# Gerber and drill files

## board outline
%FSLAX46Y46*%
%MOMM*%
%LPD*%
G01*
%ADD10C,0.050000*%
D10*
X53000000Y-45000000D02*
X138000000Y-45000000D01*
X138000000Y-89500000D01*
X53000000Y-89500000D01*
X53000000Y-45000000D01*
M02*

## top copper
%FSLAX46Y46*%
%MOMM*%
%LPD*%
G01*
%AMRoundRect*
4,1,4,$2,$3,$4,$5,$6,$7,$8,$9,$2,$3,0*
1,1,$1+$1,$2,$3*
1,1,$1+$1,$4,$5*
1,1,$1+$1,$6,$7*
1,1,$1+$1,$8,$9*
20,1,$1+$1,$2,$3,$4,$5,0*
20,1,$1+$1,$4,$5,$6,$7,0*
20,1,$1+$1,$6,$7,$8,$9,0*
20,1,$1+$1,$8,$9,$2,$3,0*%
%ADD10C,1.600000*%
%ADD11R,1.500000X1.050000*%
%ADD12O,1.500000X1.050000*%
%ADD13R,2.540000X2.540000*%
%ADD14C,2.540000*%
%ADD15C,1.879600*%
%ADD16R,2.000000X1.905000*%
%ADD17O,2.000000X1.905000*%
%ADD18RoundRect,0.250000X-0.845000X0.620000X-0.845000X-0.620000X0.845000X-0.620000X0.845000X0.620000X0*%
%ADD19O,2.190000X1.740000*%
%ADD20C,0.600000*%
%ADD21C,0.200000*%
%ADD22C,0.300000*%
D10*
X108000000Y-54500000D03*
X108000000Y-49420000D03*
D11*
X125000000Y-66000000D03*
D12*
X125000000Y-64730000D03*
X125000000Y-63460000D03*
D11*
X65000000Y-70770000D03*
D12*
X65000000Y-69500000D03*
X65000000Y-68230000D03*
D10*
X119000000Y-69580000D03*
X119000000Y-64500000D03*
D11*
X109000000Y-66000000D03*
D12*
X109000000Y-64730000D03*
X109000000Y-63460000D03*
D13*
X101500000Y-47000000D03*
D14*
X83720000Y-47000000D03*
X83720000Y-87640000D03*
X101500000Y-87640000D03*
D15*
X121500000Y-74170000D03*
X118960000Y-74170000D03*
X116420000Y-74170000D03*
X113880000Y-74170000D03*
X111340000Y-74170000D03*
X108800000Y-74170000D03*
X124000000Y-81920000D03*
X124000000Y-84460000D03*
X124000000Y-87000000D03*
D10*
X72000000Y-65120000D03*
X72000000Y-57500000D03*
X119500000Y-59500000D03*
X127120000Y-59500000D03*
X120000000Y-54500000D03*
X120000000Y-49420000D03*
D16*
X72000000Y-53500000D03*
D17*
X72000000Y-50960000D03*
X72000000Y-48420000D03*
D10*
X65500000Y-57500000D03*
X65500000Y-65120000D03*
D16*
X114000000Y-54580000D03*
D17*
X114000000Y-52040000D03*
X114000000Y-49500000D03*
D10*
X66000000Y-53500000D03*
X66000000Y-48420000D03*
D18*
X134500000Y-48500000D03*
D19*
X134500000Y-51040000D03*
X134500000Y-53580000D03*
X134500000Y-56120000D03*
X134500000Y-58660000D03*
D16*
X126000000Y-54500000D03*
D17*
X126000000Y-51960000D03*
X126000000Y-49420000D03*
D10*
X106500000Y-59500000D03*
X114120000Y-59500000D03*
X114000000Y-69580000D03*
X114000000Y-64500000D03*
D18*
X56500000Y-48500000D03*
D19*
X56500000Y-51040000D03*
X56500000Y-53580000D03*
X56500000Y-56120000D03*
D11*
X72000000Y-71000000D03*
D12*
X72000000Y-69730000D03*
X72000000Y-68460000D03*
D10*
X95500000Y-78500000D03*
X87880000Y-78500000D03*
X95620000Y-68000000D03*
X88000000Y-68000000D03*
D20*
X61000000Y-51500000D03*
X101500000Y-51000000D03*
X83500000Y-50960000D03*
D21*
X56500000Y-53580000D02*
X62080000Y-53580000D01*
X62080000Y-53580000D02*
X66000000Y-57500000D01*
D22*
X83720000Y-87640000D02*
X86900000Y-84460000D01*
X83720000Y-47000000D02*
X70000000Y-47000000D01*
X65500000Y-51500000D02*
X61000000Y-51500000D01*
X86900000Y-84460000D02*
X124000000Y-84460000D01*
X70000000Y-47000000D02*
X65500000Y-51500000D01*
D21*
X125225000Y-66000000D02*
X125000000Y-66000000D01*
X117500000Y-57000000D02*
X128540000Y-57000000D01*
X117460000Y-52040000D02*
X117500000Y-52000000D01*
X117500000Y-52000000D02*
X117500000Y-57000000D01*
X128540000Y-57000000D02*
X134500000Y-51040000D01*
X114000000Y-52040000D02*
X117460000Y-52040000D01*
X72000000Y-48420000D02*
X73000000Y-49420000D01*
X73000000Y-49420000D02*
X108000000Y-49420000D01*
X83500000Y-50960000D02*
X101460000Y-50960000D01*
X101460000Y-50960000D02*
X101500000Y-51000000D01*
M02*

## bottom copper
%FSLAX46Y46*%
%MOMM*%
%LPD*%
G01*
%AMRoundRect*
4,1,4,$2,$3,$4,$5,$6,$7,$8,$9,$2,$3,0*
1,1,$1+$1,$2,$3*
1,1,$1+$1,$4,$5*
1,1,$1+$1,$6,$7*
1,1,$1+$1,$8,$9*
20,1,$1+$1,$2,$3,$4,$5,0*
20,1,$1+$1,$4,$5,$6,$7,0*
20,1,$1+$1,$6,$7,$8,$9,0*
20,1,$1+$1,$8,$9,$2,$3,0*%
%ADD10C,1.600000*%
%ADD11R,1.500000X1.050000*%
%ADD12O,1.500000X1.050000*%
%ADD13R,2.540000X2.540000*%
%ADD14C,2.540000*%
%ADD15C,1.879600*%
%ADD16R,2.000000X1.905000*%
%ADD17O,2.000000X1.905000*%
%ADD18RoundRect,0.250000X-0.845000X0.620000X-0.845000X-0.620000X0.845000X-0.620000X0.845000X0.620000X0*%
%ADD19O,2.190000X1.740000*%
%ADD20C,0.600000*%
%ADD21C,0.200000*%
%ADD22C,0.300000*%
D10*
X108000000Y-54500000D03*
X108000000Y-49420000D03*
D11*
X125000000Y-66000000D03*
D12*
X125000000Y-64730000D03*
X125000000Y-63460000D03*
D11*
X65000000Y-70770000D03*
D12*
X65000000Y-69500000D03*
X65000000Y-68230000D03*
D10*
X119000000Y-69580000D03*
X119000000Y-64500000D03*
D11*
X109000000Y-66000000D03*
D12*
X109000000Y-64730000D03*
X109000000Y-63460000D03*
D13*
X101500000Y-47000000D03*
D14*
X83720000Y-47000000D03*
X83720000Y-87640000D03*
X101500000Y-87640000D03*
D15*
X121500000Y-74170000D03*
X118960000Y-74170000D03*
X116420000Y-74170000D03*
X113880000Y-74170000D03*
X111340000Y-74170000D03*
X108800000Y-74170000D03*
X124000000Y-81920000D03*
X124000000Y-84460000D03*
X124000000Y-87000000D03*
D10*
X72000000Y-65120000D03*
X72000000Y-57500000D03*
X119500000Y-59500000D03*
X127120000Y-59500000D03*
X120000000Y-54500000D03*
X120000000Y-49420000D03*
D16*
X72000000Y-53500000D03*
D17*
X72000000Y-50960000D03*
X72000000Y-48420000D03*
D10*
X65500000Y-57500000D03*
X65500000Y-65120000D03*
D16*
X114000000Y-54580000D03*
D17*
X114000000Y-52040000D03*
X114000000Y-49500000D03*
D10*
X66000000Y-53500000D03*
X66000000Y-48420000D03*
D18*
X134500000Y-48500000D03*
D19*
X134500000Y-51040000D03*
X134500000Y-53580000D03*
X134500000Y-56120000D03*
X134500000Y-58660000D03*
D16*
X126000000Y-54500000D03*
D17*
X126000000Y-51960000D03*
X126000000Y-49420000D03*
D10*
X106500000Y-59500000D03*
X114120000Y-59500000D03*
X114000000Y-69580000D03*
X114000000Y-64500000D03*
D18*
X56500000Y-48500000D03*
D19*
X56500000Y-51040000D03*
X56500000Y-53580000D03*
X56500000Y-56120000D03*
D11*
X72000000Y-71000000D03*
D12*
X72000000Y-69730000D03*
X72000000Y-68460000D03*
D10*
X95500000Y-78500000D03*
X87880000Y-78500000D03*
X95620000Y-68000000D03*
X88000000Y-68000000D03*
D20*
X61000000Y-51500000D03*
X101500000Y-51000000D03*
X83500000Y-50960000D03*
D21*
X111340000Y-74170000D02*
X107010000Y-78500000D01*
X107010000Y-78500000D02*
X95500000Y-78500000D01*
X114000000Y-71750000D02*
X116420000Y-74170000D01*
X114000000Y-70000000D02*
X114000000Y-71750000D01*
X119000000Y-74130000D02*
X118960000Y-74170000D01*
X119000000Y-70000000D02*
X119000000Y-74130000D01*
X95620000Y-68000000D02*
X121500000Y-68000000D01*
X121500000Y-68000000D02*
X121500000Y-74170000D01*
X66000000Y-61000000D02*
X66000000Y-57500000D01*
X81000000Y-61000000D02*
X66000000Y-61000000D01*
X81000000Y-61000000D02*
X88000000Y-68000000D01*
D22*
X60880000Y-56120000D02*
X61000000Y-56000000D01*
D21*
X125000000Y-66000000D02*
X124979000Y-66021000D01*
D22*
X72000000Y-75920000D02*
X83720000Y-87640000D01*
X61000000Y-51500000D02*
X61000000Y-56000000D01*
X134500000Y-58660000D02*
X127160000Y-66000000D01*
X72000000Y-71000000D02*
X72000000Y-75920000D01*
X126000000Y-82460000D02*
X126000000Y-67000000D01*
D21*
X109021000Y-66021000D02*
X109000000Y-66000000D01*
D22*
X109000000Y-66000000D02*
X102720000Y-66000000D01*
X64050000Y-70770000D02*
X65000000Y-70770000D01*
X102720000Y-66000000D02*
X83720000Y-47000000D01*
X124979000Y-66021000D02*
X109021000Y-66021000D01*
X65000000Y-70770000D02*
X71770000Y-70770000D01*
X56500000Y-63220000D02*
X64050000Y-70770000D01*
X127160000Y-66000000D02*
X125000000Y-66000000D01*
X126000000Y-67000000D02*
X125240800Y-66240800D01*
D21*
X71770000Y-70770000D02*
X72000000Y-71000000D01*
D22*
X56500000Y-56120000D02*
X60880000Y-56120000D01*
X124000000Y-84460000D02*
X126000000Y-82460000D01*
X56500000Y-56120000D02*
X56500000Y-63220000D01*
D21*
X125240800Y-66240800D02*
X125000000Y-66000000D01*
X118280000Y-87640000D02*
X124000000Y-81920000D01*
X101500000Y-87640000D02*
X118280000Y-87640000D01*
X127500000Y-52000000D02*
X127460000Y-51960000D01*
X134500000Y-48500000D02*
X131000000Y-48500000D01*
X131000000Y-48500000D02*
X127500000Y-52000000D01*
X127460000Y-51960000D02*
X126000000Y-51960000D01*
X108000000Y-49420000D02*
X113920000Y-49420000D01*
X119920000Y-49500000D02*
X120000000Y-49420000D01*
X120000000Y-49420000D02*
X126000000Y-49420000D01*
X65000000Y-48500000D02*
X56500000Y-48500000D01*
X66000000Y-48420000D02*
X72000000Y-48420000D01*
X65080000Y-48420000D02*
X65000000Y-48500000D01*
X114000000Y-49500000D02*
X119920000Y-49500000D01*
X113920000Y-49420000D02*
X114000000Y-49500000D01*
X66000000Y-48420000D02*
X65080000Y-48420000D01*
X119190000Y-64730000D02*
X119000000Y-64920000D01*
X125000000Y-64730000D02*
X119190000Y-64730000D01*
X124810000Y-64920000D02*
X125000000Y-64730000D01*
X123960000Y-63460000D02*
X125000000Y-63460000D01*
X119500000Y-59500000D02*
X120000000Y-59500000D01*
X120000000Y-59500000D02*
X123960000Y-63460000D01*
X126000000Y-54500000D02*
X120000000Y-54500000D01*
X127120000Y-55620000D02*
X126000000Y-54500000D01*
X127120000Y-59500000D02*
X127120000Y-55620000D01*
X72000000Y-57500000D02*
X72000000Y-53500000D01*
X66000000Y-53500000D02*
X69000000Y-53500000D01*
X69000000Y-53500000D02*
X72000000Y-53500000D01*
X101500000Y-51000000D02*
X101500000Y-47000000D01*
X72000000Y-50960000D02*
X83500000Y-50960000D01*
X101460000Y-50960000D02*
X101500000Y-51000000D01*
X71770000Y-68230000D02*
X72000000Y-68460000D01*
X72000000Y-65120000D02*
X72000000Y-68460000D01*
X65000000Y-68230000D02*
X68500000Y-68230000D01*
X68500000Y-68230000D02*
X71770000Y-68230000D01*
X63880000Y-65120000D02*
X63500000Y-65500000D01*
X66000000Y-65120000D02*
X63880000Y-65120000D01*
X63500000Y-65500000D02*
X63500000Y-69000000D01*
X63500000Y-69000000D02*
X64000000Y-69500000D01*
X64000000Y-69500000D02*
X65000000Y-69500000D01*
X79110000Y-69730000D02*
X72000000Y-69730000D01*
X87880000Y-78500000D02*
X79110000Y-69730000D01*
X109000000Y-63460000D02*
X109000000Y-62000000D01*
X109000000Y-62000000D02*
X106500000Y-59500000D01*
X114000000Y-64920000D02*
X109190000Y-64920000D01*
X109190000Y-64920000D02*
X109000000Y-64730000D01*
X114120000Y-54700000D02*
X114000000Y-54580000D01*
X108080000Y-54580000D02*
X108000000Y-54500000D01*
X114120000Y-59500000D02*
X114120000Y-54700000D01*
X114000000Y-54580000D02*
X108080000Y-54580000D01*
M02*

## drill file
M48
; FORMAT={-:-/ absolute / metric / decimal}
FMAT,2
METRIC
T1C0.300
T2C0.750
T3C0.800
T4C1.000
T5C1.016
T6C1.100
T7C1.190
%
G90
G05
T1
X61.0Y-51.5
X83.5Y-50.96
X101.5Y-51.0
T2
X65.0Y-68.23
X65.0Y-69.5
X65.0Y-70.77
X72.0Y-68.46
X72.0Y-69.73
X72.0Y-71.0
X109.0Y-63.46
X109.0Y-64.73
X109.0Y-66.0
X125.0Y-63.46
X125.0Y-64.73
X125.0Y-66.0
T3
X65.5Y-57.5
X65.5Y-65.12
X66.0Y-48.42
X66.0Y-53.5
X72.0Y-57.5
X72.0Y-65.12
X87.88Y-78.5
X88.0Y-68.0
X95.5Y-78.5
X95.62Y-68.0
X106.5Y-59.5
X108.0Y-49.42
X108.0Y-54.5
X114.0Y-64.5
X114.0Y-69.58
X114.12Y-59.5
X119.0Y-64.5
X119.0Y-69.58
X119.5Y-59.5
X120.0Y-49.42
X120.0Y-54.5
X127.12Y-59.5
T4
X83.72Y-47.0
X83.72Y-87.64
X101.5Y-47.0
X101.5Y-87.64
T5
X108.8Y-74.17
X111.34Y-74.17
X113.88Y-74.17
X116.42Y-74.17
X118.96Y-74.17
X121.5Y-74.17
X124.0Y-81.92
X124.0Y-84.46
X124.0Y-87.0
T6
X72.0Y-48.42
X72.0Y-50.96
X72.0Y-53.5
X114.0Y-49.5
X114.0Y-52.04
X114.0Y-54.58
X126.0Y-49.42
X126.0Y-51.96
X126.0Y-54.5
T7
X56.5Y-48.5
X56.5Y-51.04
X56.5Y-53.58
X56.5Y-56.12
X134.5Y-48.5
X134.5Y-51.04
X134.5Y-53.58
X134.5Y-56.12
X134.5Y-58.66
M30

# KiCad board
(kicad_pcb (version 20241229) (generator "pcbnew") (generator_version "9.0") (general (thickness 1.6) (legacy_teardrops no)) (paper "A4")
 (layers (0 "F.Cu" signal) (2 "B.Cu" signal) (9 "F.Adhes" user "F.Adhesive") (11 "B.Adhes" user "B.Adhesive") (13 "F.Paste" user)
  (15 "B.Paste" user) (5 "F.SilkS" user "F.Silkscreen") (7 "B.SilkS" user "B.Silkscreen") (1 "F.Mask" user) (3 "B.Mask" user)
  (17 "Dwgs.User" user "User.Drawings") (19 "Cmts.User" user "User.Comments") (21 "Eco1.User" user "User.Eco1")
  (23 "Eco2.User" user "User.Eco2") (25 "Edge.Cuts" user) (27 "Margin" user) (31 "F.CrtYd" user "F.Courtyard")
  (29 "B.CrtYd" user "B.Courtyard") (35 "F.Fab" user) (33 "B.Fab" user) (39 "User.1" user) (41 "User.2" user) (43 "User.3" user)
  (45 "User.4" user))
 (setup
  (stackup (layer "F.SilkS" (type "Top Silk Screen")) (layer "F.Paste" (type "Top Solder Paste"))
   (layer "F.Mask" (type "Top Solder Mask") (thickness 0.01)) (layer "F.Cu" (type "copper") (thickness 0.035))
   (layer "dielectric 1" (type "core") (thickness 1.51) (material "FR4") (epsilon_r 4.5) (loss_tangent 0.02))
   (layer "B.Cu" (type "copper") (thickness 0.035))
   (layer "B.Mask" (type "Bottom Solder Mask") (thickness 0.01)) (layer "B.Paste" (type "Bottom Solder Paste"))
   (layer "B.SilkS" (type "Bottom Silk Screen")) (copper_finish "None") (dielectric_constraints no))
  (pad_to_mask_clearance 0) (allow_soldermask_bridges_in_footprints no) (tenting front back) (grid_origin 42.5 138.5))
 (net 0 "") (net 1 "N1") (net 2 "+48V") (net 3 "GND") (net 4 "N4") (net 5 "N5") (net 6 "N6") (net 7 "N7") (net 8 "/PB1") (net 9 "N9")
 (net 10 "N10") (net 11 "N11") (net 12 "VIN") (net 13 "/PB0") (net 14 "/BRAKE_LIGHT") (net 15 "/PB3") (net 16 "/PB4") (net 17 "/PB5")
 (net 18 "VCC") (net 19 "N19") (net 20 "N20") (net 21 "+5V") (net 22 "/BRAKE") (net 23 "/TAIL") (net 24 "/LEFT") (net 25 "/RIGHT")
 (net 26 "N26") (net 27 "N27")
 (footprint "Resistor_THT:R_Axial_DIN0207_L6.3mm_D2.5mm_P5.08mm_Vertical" (layer "F.Cu") (at 108 54.5 90)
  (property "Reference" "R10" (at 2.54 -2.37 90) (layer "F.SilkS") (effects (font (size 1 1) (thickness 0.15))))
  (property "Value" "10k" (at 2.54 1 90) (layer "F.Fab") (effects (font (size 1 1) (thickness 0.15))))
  (pad "1" thru_hole circle (at 0 0 90) (size 1.6 1.6) (drill 0.8) (layers "*.Cu" "*.Mask") (remove_unused_layers no) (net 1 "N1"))
  (pad "2" thru_hole circle (at 5.08 0 90) (size 1.6 1.6) (drill 0.8) (layers "*.Cu" "*.Mask") (remove_unused_layers no) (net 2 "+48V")))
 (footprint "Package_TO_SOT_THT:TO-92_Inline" (layer "F.Cu") (at 125 66 90)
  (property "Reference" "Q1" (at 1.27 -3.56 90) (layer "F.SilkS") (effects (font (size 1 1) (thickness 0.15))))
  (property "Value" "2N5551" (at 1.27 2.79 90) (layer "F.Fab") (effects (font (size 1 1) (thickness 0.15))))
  (pad "1" thru_hole rect (at 0 0 90) (size 1.05 1.5) (drill 0.75) (layers "*.Cu" "*.Mask") (remove_unused_layers no) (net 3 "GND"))
  (pad "2" thru_hole oval (at 1.27 0 90) (size 1.05 1.5) (drill 0.75) (layers "*.Cu" "*.Mask") (remove_unused_layers no) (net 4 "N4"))
  (pad "3" thru_hole oval (at 2.54 0 90) (size 1.05 1.5) (drill 0.75) (layers "*.Cu" "*.Mask") (remove_unused_layers no) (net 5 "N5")))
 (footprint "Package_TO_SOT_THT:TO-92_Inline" (layer "F.Cu") (at 65 70.77 90)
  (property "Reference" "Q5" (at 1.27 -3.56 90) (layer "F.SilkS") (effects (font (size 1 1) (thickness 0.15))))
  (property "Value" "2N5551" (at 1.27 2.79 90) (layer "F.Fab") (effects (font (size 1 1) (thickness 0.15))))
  (pad "1" thru_hole rect (at 0 0 90) (size 1.05 1.5) (drill 0.75) (layers "*.Cu" "*.Mask") (remove_unused_layers no) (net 3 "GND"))
  (pad "2" thru_hole oval (at 1.27 0 90) (size 1.05 1.5) (drill 0.75) (layers "*.Cu" "*.Mask") (remove_unused_layers no) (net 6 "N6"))
  (pad "3" thru_hole oval (at 2.54 0 90) (size 1.05 1.5) (drill 0.75) (layers "*.Cu" "*.Mask") (remove_unused_layers no) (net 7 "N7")))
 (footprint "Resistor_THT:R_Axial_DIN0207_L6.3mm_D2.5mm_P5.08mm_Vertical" (layer "F.Cu") (at 119 69.58 90)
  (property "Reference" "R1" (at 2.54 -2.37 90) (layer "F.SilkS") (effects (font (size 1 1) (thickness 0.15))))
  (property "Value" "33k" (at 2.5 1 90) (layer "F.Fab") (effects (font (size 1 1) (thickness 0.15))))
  (pad "1" thru_hole circle (at 0 0 90) (size 1.6 1.6) (drill 0.8) (layers "*.Cu" "*.Mask") (remove_unused_layers no) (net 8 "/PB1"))
  (pad "2" thru_hole circle (at 5.08 0 90) (size 1.6 1.6) (drill 0.8) (layers "*.Cu" "*.Mask") (remove_unused_layers no) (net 4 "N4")))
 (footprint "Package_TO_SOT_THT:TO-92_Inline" (layer "F.Cu") (at 109 66 90)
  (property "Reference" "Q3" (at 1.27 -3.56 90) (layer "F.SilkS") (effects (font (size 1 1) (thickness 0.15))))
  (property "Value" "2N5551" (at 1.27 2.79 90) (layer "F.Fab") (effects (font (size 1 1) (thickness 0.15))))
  (pad "1" thru_hole rect (at 0 0 90) (size 1.05 1.5) (drill 0.75) (layers "*.Cu" "*.Mask") (remove_unused_layers no) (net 3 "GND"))
  (pad "2" thru_hole oval (at 1.27 0 90) (size 1.05 1.5) (drill 0.75) (layers "*.Cu" "*.Mask") (remove_unused_layers no) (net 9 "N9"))
  (pad "3" thru_hole oval (at 2.54 0 90) (size 1.05 1.5) (drill 0.75) (layers "*.Cu" "*.Mask") (remove_unused_layers no) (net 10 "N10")))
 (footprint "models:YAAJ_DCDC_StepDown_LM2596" (layer "F.Cu") (at 101.5 47 -90)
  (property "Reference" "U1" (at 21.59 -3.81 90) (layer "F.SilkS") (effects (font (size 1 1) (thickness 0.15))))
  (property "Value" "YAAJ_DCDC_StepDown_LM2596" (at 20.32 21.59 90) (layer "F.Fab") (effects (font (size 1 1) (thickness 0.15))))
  (pad "1" thru_hole rect (at 0 0 270) (size 2.54 2.54) (drill 1) (layers "*.Cu" "*.Mask") (remove_unused_layers no) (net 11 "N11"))
  (pad "2" thru_hole circle (at 0 17.78 270) (size 2.54 2.54) (drill 1) (layers "*.Cu" "*.Mask") (remove_unused_layers no) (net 3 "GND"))
  (pad "3" thru_hole circle (at 40.64 17.78 270) (size 2.54 2.54) (drill 1) (layers "*.Cu" "*.Mask") (remove_unused_layers no) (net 3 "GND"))
  (pad "4" thru_hole circle (at 40.64 0 270) (size 2.54 2.54) (drill 1) (layers "*.Cu" "*.Mask") (remove_unused_layers no) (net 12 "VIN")))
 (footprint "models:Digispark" (layer "F.Cu") (at 115.15 74.17 180)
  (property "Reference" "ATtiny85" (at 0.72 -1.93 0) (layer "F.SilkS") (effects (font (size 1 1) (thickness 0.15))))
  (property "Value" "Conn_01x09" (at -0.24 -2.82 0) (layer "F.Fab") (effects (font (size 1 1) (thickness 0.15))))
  (pad "1" thru_hole circle (at -6.35 0 180) (size 1.8796 1.8796) (drill 1.016) (layers "*.Cu" "*.Mask") (remove_unused_layers no)
   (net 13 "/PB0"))
  (pad "2" thru_hole circle (at -3.81 0 180) (size 1.8796 1.8796) (drill 1.016) (layers "*.Cu" "*.Mask") (remove_unused_layers no)
   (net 8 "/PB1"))
  (pad "3" thru_hole circle (at -1.27 0 180) (size 1.8796 1.8796) (drill 1.016) (layers "*.Cu" "*.Mask") (remove_unused_layers no)
   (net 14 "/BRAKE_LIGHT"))
  (pad "4" thru_hole circle (at 1.27 0 180) (size 1.8796 1.8796) (drill 1.016) (layers "*.Cu" "*.Mask") (remove_unused_layers no)
   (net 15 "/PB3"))
  (pad "5" thru_hole circle (at 3.81 0 180) (size 1.8796 1.8796) (drill 1.016) (layers "*.Cu" "*.Mask") (remove_unused_layers no)
   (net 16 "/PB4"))
  (pad "6" thru_hole circle (at 6.35 0 180) (size 1.8796 1.8796) (drill 1.016) (layers "*.Cu" "*.Mask") (remove_unused_layers no)
   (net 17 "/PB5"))
  (pad "7" thru_hole circle (at -8.85 -7.75 180) (size 1.8796 1.8796) (drill 1.016) (layers "*.Cu" "*.Mask") (remove_unused_layers no)
   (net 12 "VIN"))
  (pad "8" thru_hole circle (at -8.85 -10.29 180) (size 1.8796 1.8796) (drill 1.016) (layers "*.Cu" "*.Mask") (remove_unused_layers no)
   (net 3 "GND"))
  (pad "9" thru_hole circle (at -8.85 -12.83 180) (size 1.8796 1.8796) (drill 1.016) (layers "*.Cu" "*.Mask") (remove_unused_layers no)
   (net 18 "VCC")))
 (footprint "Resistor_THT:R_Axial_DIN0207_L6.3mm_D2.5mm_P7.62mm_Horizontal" (layer "F.Cu") (at 72 65.12 90)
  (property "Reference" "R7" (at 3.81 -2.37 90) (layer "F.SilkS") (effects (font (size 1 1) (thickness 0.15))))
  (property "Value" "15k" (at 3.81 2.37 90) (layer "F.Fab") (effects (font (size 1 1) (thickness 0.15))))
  (pad "1" thru_hole circle (at 0 0 90) (size 1.6 1.6) (drill 0.8) (layers "*.Cu" "*.Mask") (remove_unused_layers no) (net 7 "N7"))
  (pad "2" thru_hole circle (at 7.62 0 90) (size 1.6 1.6) (drill 0.8) (layers "*.Cu" "*.Mask") (remove_unused_layers no) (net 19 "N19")))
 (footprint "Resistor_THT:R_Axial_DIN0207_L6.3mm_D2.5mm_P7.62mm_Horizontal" (layer "F.Cu") (at 119.5 59.5)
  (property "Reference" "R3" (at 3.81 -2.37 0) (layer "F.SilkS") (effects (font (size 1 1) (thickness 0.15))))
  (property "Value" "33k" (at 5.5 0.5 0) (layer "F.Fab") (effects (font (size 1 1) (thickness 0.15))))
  (pad "1" thru_hole circle (at 0 0) (size 1.6 1.6) (drill 0.8) (layers "*.Cu" "*.Mask") (remove_unused_layers no) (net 5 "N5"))
  (pad "2" thru_hole circle (at 7.62 0) (size 1.6 1.6) (drill 0.8) (layers "*.Cu" "*.Mask") (remove_unused_layers no) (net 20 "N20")))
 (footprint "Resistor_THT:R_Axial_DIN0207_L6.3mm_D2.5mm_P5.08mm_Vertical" (layer "F.Cu") (at 120 54.5 90)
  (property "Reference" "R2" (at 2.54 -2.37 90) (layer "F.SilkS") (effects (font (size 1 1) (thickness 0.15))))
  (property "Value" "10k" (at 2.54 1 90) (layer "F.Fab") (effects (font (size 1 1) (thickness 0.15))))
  (pad "1" thru_hole circle (at 0 0 90) (size 1.6 1.6) (drill 0.8) (layers "*.Cu" "*.Mask") (remove_unused_layers no) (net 20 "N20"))
  (pad "2" thru_hole circle (at 5.08 0 90) (size 1.6 1.6) (drill 0.8) (layers "*.Cu" "*.Mask") (remove_unused_layers no) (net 2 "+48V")))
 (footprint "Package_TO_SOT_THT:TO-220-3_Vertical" (layer "F.Cu") (at 72 53.5 90)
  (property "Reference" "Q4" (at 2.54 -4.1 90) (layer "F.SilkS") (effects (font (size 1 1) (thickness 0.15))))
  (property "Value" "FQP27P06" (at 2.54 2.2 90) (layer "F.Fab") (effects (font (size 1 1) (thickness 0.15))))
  (pad "1" thru_hole rect (at 0 0 90) (size 1.905 2) (drill 1.1) (layers "*.Cu" "*.Mask") (remove_unused_layers no) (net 19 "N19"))
  (pad "2" thru_hole oval (at 2.54 0 90) (size 1.905 2) (drill 1.1) (layers "*.Cu" "*.Mask") (remove_unused_layers no) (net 11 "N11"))
  (pad "3" thru_hole oval (at 5.08 0 90) (size 1.905 2) (drill 1.1) (layers "*.Cu" "*.Mask") (remove_unused_layers no) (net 2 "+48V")))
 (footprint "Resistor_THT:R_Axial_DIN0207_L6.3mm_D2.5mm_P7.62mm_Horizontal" (layer "F.Cu") (at 65.5 57.5 -90)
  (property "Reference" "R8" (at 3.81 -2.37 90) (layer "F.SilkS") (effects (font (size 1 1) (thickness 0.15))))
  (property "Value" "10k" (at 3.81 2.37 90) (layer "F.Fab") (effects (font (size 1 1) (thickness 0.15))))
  (pad "1" thru_hole circle (at 0 0 270) (size 1.6 1.6) (drill 0.8) (layers "*.Cu" "*.Mask") (remove_unused_layers no) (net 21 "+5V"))
  (pad "2" thru_hole circle (at 7.62 0 270) (size 1.6 1.6) (drill 0.8) (layers "*.Cu" "*.Mask") (remove_unused_layers no) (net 6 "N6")))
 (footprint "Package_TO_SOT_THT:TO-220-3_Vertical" (layer "F.Cu") (at 114 54.58 90)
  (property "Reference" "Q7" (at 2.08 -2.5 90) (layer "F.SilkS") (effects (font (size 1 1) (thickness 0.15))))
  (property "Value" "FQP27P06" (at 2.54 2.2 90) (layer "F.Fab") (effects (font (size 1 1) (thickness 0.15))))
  (pad "1" thru_hole rect (at 0 0 90) (size 1.905 2) (drill 1.1) (layers "*.Cu" "*.Mask") (remove_unused_layers no) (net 1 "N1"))
  (pad "2" thru_hole oval (at 2.54 0 90) (size 1.905 2) (drill 1.1) (layers "*.Cu" "*.Mask") (remove_unused_layers no) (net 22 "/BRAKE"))
  (pad "3" thru_hole oval (at 5.08 0 90) (size 1.905 2) (drill 1.1) (layers "*.Cu" "*.Mask") (remove_unused_layers no) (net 2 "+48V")))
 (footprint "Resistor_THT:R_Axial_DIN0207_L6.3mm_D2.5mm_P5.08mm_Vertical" (layer "F.Cu") (at 66 53.5 90)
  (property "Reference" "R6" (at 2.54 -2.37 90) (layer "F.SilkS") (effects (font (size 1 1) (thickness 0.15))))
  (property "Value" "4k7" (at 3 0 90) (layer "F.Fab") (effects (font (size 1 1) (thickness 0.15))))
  (pad "1" thru_hole circle (at 0 0 90) (size 1.6 1.6) (drill 0.8) (layers "*.Cu" "*.Mask") (remove_unused_layers no) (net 19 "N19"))
  (pad "2" thru_hole circle (at 5.08 0 90) (size 1.6 1.6) (drill 0.8) (layers "*.Cu" "*.Mask") (remove_unused_layers no) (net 2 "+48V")))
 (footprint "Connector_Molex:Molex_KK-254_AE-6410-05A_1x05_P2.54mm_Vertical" (layer "F.Cu") (at 134.5 48.5 -90)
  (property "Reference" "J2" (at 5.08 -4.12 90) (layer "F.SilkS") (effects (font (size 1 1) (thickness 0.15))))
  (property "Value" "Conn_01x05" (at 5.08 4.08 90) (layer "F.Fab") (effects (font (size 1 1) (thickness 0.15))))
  (pad "1" thru_hole roundrect (at 0 0 270) (size 1.74 2.19) (drill 1.19) (layers "*.Cu" "*.Mask") (remove_unused_layers no)
   (roundrect_rratio 0.143678) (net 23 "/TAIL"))
  (pad "2" thru_hole oval (at 2.54 0 270) (size 1.74 2.19) (drill 1.19) (layers "*.Cu" "*.Mask") (remove_unused_layers no) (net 22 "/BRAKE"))
  (pad "3" thru_hole oval (at 5.08 0 270) (size 1.74 2.19) (drill 1.19) (layers "*.Cu" "*.Mask") (remove_unused_layers no) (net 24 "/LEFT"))
  (pad "4" thru_hole oval (at 7.62 0 270) (size 1.74 2.19) (drill 1.19) (layers "*.Cu" "*.Mask") (remove_unused_layers no) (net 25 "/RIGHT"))
  (pad "5" thru_hole oval (at 10.16 0 270) (size 1.74 2.19) (drill 1.19) (layers "*.Cu" "*.Mask") (remove_unused_layers no) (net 3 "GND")))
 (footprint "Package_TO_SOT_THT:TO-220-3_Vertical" (layer "F.Cu") (at 126 54.5 90)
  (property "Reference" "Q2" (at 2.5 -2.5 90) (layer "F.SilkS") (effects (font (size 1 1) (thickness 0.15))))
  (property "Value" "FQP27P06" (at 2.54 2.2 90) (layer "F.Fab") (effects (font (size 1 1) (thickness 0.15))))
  (pad "1" thru_hole rect (at 0 0 90) (size 1.905 2) (drill 1.1) (layers "*.Cu" "*.Mask") (remove_unused_layers no) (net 20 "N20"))
  (pad "2" thru_hole oval (at 2.54 0 90) (size 1.905 2) (drill 1.1) (layers "*.Cu" "*.Mask") (remove_unused_layers no) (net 23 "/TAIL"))
  (pad "3" thru_hole oval (at 5.08 0 90) (size 1.905 2) (drill 1.1) (layers "*.Cu" "*.Mask") (remove_unused_layers no) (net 2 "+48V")))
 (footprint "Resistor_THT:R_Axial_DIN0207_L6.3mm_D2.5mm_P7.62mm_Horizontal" (layer "F.Cu") (at 106.5 59.5)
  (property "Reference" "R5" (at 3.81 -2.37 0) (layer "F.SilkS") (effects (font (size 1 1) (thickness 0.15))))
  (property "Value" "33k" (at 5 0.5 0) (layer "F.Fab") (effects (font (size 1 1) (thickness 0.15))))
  (pad "1" thru_hole circle (at 0 0) (size 1.6 1.6) (drill 0.8) (layers "*.Cu" "*.Mask") (remove_unused_layers no) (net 10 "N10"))
  (pad "2" thru_hole circle (at 7.62 0) (size 1.6 1.6) (drill 0.8) (layers "*.Cu" "*.Mask") (remove_unused_layers no) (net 1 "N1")))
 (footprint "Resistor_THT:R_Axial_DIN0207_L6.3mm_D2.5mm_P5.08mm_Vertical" (layer "F.Cu") (at 114 69.58 90)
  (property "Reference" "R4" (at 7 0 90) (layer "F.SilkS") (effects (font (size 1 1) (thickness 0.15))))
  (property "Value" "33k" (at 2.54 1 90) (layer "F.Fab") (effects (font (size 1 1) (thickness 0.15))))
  (pad "1" thru_hole circle (at 0 0 90) (size 1.6 1.6) (drill 0.8) (layers "*.Cu" "*.Mask") (remove_unused_layers no)
   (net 14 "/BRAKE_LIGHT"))
  (pad "2" thru_hole circle (at 5.08 0 90) (size 1.6 1.6) (drill 0.8) (layers "*.Cu" "*.Mask") (remove_unused_layers no) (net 9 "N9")))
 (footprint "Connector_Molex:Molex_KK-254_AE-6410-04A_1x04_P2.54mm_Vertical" (layer "F.Cu") (at 56.5 48.5 -90)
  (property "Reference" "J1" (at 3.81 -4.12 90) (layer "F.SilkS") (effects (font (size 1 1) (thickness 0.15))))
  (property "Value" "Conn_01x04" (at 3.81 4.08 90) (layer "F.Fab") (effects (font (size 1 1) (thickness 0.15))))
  (pad "1" thru_hole roundrect (at 0 0 270) (size 1.74 2.19) (drill 1.19) (layers "*.Cu" "*.Mask") (remove_unused_layers no)
   (roundrect_rratio 0.143678) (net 2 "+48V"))
  (pad "2" thru_hole oval (at 2.54 0 270) (size 1.74 2.19) (drill 1.19) (layers "*.Cu" "*.Mask") (remove_unused_layers no) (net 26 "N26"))
  (pad "3" thru_hole oval (at 5.08 0 270) (size 1.74 2.19) (drill 1.19) (layers "*.Cu" "*.Mask") (remove_unused_layers no) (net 21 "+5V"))
  (pad "4" thru_hole oval (at 7.62 0 270) (size 1.74 2.19) (drill 1.19) (layers "*.Cu" "*.Mask") (remove_unused_layers no) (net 3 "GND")))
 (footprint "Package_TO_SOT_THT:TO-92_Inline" (layer "F.Cu") (at 72 71 90)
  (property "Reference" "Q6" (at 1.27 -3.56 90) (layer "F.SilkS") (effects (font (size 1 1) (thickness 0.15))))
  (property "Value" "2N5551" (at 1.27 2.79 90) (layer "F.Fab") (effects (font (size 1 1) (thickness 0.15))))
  (pad "1" thru_hole rect (at 0 0 90) (size 1.05 1.5) (drill 0.75) (layers "*.Cu" "*.Mask") (remove_unused_layers no) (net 3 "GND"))
  (pad "2" thru_hole oval (at 1.27 0 90) (size 1.05 1.5) (drill 0.75) (layers "*.Cu" "*.Mask") (remove_unused_layers no) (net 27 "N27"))
  (pad "3" thru_hole oval (at 2.54 0 90) (size 1.05 1.5) (drill 0.75) (layers "*.Cu" "*.Mask") (remove_unused_layers no) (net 7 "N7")))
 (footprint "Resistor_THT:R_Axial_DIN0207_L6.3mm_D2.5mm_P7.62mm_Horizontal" (layer "B.Cu") (at 95.5 78.5 180)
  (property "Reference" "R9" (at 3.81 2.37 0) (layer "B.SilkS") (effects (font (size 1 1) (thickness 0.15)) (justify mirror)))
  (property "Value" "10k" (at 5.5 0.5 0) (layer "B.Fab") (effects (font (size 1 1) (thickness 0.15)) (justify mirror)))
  (pad "1" thru_hole circle (at 0 0 180) (size 1.6 1.6) (drill 0.8) (layers "*.Cu" "*.Mask") (remove_unused_layers no) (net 16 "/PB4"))
  (pad "2" thru_hole circle (at 7.62 0 180) (size 1.6 1.6) (drill 0.8) (layers "*.Cu" "*.Mask") (remove_unused_layers no) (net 27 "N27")))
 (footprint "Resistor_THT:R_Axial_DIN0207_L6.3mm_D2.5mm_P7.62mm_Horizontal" (layer "B.Cu") (at 95.62 68 180)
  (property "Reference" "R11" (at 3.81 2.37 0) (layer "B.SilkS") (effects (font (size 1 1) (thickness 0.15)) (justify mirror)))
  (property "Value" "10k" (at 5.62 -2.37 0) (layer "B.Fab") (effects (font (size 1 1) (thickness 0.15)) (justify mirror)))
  (pad "1" thru_hole circle (at 0 0 180) (size 1.6 1.6) (drill 0.8) (layers "*.Cu" "*.Mask") (remove_unused_layers no) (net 13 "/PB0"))
  (pad "2" thru_hole circle (at 7.62 0 180) (size 1.6 1.6) (drill 0.8) (layers "*.Cu" "*.Mask") (remove_unused_layers no) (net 21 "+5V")))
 (gr_rect (start 53 45) (end 138 89.5) (stroke (width 0.05) (type default)) (fill no) (layer "Edge.Cuts"))
 (segment (start 111.34 74.17) (end 107.01 78.5) (width 0.2) (layer "B.Cu") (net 16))
 (segment (start 107.01 78.5) (end 95.5 78.5) (width 0.2) (layer "B.Cu") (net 16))
 (segment (start 114 71.75) (end 116.42 74.17) (width 0.2) (layer "B.Cu") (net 14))
 (segment (start 114 70) (end 114 71.75) (width 0.2) (layer "B.Cu") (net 14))
 (segment (start 119 74.13) (end 118.96 74.17) (width 0.2) (layer "B.Cu") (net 8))
 (segment (start 119 70) (end 119 74.13) (width 0.2) (layer "B.Cu") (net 8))
 (segment (start 95.62 68) (end 121.5 68) (width 0.2) (layer "B.Cu") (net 13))
 (segment (start 121.5 68) (end 121.5 74.17) (width 0.2) (layer "B.Cu") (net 13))
 (segment (start 56.5 53.58) (end 62.08 53.58) (width 0.2) (layer "F.Cu") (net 21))
 (segment (start 62.08 53.58) (end 66 57.5) (width 0.2) (layer "F.Cu") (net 21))
 (segment (start 66 61) (end 66 57.5) (width 0.2) (layer "B.Cu") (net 21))
 (segment (start 81 61) (end 66 61) (width 0.2) (layer "B.Cu") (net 21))
 (segment (start 81 61) (end 88 68) (width 0.2) (layer "B.Cu") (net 21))
 (segment (start 83.72 87.64) (end 86.9 84.46) (width 0.3) (layer "F.Cu") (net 3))
 (segment (start 83.72 47) (end 70 47) (width 0.3) (layer "F.Cu") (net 3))
 (segment (start 65.5 51.5) (end 61 51.5) (width 0.3) (layer "F.Cu") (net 3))
 (segment (start 86.9 84.46) (end 124 84.46) (width 0.3) (layer "F.Cu") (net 3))
 (segment (start 70 47) (end 65.5 51.5) (width 0.3) (layer "F.Cu") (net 3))
 (segment (start 125.225 66) (end 125 66) (width 0.2) (layer "F.Cu") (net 3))
 (via (at 61 51.5) (size 0.6) (drill 0.3) (layers "F.Cu" "B.Cu") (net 3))
 (segment (start 60.88 56.12) (end 61 56) (width 0.3) (layer "B.Cu") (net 3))
 (segment (start 125 66) (end 124.979 66.021) (width 0.2) (layer "B.Cu") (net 3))
 (segment (start 72 75.92) (end 83.72 87.64) (width 0.3) (layer "B.Cu") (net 3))
 (segment (start 61 51.5) (end 61 56) (width 0.3) (layer "B.Cu") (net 3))
 (segment (start 134.5 58.66) (end 127.16 66) (width 0.3) (layer "B.Cu") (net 3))
 (segment (start 72 71) (end 72 75.92) (width 0.3) (layer "B.Cu") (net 3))
 (segment (start 126 82.46) (end 126 67) (width 0.3) (layer "B.Cu") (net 3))
 (segment (start 109.021 66.021) (end 109 66) (width 0.2) (layer "B.Cu") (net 3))
 (segment (start 109 66) (end 102.72 66) (width 0.3) (layer "B.Cu") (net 3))
 (segment (start 64.05 70.77) (end 65 70.77) (width 0.3) (layer "B.Cu") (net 3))
 (segment (start 102.72 66) (end 83.72 47) (width 0.3) (layer "B.Cu") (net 3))
 (segment (start 124.979 66.021) (end 109.021 66.021) (width 0.3) (layer "B.Cu") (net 3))
 (segment (start 65 70.77) (end 71.77 70.77) (width 0.3) (layer "B.Cu") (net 3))
 (segment (start 56.5 63.22) (end 64.05 70.77) (width 0.3) (layer "B.Cu") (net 3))
 (segment (start 127.16 66) (end 125 66) (width 0.3) (layer "B.Cu") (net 3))
 (segment (start 126 67) (end 125.2408 66.2408) (width 0.3) (layer "B.Cu") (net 3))
 (segment (start 71.77 70.77) (end 72 71) (width 0.2) (layer "B.Cu") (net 3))
 (segment (start 56.5 56.12) (end 60.88 56.12) (width 0.3) (layer "B.Cu") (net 3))
 (segment (start 124 84.46) (end 126 82.46) (width 0.3) (layer "B.Cu") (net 3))
 (segment (start 56.5 56.12) (end 56.5 63.22) (width 0.3) (layer "B.Cu") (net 3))
 (segment (start 125.2408 66.2408) (end 125 66) (width 0.2) (layer "B.Cu") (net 3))
 (segment (start 118.28 87.64) (end 124 81.92) (width 0.2) (layer "B.Cu") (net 12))
 (segment (start 101.5 87.64) (end 118.28 87.64) (width 0.2) (layer "B.Cu") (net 12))
 (segment (start 127.5 52) (end 127.46 51.96) (width 0.2) (layer "B.Cu") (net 23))
 (segment (start 134.5 48.5) (end 131 48.5) (width 0.2) (layer "B.Cu") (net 23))
 (segment (start 131 48.5) (end 127.5 52) (width 0.2) (layer "B.Cu") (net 23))
 (segment (start 127.46 51.96) (end 126 51.96) (width 0.2) (layer "B.Cu") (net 23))
 (segment (start 117.5 57) (end 128.54 57) (width 0.2) (layer "F.Cu") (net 22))
 (segment (start 117.46 52.04) (end 117.5 52) (width 0.2) (layer "F.Cu") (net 22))
 (segment (start 117.5 52) (end 117.5 57) (width 0.2) (layer "F.Cu") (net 22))
 (segment (start 128.54 57) (end 134.5 51.04) (width 0.2) (layer "F.Cu") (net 22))
 (segment (start 114 52.04) (end 117.46 52.04) (width 0.2) (layer "F.Cu") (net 22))
 (segment (start 72 48.42) (end 73 49.42) (width 0.2) (layer "F.Cu") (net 2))
 (segment (start 73 49.42) (end 108 49.42) (width 0.2) (layer "F.Cu") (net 2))
 (segment (start 108 49.42) (end 113.92 49.42) (width 0.2) (layer "B.Cu") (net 2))
 (segment (start 119.92 49.5) (end 120 49.42) (width 0.2) (layer "B.Cu") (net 2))
 (segment (start 120 49.42) (end 126 49.42) (width 0.2) (layer "B.Cu") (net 2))
 (segment (start 65 48.5) (end 56.5 48.5) (width 0.2) (layer "B.Cu") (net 2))
 (segment (start 66 48.42) (end 72 48.42) (width 0.2) (layer "B.Cu") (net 2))
 (segment (start 65.08 48.42) (end 65 48.5) (width 0.2) (layer "B.Cu") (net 2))
 (segment (start 114 49.5) (end 119.92 49.5) (width 0.2) (layer "B.Cu") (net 2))
 (segment (start 113.92 49.42) (end 114 49.5) (width 0.2) (layer "B.Cu") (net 2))
 (segment (start 66 48.42) (end 65.08 48.42) (width 0.2) (layer "B.Cu") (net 2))
 (segment (start 119.19 64.73) (end 119 64.92) (width 0.2) (layer "B.Cu") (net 4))
 (segment (start 125 64.73) (end 119.19 64.73) (width 0.2) (layer "B.Cu") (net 4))
 (segment (start 124.81 64.92) (end 125 64.73) (width 0.2) (layer "B.Cu") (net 4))
 (segment (start 123.96 63.46) (end 125 63.46) (width 0.2) (layer "B.Cu") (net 5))
 (segment (start 119.5 59.5) (end 120 59.5) (width 0.2) (layer "B.Cu") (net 5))
 (segment (start 120 59.5) (end 123.96 63.46) (width 0.2) (layer "B.Cu") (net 5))
 (segment (start 126 54.5) (end 120 54.5) (width 0.2) (layer "B.Cu") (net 20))
 (segment (start 127.12 55.62) (end 126 54.5) (width 0.2) (layer "B.Cu") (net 20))
 (segment (start 127.12 59.5) (end 127.12 55.62) (width 0.2) (layer "B.Cu") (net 20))
 (segment (start 72 57.5) (end 72 53.5) (width 0.2) (layer "B.Cu") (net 19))
 (segment (start 66 53.5) (end 69 53.5) (width 0.2) (layer "B.Cu") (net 19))
 (segment (start 69 53.5) (end 72 53.5) (width 0.2) (layer "B.Cu") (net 19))
 (segment (start 83.5 50.96) (end 101.46 50.96) (width 0.2) (layer "F.Cu") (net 11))
 (segment (start 101.46 50.96) (end 101.5 51) (width 0.2) (layer "F.Cu") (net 11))
 (via (at 101.5 51) (size 0.6) (drill 0.3) (layers "F.Cu" "B.Cu") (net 11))
 (via (at 83.5 50.96) (size 0.6) (drill 0.3) (layers "F.Cu" "B.Cu") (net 11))
 (segment (start 101.5 51) (end 101.5 47) (width 0.2) (layer "B.Cu") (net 11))
 (segment (start 72 50.96) (end 83.5 50.96) (width 0.2) (layer "B.Cu") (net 11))
 (segment (start 101.46 50.96) (end 101.5 51) (width 0.2) (layer "B.Cu") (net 11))
 (segment (start 71.77 68.23) (end 72 68.46) (width 0.2) (layer "B.Cu") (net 7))
 (segment (start 72 65.12) (end 72 68.46) (width 0.2) (layer "B.Cu") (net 7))
 (segment (start 65 68.23) (end 68.5 68.23) (width 0.2) (layer "B.Cu") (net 7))
 (segment (start 68.5 68.23) (end 71.77 68.23) (width 0.2) (layer "B.Cu") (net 7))
 (segment (start 63.88 65.12) (end 63.5 65.5) (width 0.2) (layer "B.Cu") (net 6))
 (segment (start 66 65.12) (end 63.88 65.12) (width 0.2) (layer "B.Cu") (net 6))
 (segment (start 63.5 65.5) (end 63.5 69) (width 0.2) (layer "B.Cu") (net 6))
 (segment (start 63.5 69) (end 64 69.5) (width 0.2) (layer "B.Cu") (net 6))
 (segment (start 64 69.5) (end 65 69.5) (width 0.2) (layer "B.Cu") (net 6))
 (segment (start 79.11 69.73) (end 72 69.73) (width 0.2) (layer "B.Cu") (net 27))
 (segment (start 87.88 78.5) (end 79.11 69.73) (width 0.2) (layer "B.Cu") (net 27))
 (segment (start 109 63.46) (end 109 62) (width 0.2) (layer "B.Cu") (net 10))
 (segment (start 109 62) (end 106.5 59.5) (width 0.2) (layer "B.Cu") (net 10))
 (segment (start 114 64.92) (end 109.19 64.92) (width 0.2) (layer "B.Cu") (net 9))
 (segment (start 109.19 64.92) (end 109 64.73) (width 0.2) (layer "B.Cu") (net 9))
 (segment (start 114.12 54.7) (end 114 54.58) (width 0.2) (layer "B.Cu") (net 1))
 (segment (start 108.08 54.58) (end 108 54.5) (width 0.2) (layer "B.Cu") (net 1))
 (segment (start 114.12 59.5) (end 114.12 54.7) (width 0.2) (layer "B.Cu") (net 1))
 (segment (start 114 54.58) (end 108.08 54.58) (width 0.2) (layer "B.Cu") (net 1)))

